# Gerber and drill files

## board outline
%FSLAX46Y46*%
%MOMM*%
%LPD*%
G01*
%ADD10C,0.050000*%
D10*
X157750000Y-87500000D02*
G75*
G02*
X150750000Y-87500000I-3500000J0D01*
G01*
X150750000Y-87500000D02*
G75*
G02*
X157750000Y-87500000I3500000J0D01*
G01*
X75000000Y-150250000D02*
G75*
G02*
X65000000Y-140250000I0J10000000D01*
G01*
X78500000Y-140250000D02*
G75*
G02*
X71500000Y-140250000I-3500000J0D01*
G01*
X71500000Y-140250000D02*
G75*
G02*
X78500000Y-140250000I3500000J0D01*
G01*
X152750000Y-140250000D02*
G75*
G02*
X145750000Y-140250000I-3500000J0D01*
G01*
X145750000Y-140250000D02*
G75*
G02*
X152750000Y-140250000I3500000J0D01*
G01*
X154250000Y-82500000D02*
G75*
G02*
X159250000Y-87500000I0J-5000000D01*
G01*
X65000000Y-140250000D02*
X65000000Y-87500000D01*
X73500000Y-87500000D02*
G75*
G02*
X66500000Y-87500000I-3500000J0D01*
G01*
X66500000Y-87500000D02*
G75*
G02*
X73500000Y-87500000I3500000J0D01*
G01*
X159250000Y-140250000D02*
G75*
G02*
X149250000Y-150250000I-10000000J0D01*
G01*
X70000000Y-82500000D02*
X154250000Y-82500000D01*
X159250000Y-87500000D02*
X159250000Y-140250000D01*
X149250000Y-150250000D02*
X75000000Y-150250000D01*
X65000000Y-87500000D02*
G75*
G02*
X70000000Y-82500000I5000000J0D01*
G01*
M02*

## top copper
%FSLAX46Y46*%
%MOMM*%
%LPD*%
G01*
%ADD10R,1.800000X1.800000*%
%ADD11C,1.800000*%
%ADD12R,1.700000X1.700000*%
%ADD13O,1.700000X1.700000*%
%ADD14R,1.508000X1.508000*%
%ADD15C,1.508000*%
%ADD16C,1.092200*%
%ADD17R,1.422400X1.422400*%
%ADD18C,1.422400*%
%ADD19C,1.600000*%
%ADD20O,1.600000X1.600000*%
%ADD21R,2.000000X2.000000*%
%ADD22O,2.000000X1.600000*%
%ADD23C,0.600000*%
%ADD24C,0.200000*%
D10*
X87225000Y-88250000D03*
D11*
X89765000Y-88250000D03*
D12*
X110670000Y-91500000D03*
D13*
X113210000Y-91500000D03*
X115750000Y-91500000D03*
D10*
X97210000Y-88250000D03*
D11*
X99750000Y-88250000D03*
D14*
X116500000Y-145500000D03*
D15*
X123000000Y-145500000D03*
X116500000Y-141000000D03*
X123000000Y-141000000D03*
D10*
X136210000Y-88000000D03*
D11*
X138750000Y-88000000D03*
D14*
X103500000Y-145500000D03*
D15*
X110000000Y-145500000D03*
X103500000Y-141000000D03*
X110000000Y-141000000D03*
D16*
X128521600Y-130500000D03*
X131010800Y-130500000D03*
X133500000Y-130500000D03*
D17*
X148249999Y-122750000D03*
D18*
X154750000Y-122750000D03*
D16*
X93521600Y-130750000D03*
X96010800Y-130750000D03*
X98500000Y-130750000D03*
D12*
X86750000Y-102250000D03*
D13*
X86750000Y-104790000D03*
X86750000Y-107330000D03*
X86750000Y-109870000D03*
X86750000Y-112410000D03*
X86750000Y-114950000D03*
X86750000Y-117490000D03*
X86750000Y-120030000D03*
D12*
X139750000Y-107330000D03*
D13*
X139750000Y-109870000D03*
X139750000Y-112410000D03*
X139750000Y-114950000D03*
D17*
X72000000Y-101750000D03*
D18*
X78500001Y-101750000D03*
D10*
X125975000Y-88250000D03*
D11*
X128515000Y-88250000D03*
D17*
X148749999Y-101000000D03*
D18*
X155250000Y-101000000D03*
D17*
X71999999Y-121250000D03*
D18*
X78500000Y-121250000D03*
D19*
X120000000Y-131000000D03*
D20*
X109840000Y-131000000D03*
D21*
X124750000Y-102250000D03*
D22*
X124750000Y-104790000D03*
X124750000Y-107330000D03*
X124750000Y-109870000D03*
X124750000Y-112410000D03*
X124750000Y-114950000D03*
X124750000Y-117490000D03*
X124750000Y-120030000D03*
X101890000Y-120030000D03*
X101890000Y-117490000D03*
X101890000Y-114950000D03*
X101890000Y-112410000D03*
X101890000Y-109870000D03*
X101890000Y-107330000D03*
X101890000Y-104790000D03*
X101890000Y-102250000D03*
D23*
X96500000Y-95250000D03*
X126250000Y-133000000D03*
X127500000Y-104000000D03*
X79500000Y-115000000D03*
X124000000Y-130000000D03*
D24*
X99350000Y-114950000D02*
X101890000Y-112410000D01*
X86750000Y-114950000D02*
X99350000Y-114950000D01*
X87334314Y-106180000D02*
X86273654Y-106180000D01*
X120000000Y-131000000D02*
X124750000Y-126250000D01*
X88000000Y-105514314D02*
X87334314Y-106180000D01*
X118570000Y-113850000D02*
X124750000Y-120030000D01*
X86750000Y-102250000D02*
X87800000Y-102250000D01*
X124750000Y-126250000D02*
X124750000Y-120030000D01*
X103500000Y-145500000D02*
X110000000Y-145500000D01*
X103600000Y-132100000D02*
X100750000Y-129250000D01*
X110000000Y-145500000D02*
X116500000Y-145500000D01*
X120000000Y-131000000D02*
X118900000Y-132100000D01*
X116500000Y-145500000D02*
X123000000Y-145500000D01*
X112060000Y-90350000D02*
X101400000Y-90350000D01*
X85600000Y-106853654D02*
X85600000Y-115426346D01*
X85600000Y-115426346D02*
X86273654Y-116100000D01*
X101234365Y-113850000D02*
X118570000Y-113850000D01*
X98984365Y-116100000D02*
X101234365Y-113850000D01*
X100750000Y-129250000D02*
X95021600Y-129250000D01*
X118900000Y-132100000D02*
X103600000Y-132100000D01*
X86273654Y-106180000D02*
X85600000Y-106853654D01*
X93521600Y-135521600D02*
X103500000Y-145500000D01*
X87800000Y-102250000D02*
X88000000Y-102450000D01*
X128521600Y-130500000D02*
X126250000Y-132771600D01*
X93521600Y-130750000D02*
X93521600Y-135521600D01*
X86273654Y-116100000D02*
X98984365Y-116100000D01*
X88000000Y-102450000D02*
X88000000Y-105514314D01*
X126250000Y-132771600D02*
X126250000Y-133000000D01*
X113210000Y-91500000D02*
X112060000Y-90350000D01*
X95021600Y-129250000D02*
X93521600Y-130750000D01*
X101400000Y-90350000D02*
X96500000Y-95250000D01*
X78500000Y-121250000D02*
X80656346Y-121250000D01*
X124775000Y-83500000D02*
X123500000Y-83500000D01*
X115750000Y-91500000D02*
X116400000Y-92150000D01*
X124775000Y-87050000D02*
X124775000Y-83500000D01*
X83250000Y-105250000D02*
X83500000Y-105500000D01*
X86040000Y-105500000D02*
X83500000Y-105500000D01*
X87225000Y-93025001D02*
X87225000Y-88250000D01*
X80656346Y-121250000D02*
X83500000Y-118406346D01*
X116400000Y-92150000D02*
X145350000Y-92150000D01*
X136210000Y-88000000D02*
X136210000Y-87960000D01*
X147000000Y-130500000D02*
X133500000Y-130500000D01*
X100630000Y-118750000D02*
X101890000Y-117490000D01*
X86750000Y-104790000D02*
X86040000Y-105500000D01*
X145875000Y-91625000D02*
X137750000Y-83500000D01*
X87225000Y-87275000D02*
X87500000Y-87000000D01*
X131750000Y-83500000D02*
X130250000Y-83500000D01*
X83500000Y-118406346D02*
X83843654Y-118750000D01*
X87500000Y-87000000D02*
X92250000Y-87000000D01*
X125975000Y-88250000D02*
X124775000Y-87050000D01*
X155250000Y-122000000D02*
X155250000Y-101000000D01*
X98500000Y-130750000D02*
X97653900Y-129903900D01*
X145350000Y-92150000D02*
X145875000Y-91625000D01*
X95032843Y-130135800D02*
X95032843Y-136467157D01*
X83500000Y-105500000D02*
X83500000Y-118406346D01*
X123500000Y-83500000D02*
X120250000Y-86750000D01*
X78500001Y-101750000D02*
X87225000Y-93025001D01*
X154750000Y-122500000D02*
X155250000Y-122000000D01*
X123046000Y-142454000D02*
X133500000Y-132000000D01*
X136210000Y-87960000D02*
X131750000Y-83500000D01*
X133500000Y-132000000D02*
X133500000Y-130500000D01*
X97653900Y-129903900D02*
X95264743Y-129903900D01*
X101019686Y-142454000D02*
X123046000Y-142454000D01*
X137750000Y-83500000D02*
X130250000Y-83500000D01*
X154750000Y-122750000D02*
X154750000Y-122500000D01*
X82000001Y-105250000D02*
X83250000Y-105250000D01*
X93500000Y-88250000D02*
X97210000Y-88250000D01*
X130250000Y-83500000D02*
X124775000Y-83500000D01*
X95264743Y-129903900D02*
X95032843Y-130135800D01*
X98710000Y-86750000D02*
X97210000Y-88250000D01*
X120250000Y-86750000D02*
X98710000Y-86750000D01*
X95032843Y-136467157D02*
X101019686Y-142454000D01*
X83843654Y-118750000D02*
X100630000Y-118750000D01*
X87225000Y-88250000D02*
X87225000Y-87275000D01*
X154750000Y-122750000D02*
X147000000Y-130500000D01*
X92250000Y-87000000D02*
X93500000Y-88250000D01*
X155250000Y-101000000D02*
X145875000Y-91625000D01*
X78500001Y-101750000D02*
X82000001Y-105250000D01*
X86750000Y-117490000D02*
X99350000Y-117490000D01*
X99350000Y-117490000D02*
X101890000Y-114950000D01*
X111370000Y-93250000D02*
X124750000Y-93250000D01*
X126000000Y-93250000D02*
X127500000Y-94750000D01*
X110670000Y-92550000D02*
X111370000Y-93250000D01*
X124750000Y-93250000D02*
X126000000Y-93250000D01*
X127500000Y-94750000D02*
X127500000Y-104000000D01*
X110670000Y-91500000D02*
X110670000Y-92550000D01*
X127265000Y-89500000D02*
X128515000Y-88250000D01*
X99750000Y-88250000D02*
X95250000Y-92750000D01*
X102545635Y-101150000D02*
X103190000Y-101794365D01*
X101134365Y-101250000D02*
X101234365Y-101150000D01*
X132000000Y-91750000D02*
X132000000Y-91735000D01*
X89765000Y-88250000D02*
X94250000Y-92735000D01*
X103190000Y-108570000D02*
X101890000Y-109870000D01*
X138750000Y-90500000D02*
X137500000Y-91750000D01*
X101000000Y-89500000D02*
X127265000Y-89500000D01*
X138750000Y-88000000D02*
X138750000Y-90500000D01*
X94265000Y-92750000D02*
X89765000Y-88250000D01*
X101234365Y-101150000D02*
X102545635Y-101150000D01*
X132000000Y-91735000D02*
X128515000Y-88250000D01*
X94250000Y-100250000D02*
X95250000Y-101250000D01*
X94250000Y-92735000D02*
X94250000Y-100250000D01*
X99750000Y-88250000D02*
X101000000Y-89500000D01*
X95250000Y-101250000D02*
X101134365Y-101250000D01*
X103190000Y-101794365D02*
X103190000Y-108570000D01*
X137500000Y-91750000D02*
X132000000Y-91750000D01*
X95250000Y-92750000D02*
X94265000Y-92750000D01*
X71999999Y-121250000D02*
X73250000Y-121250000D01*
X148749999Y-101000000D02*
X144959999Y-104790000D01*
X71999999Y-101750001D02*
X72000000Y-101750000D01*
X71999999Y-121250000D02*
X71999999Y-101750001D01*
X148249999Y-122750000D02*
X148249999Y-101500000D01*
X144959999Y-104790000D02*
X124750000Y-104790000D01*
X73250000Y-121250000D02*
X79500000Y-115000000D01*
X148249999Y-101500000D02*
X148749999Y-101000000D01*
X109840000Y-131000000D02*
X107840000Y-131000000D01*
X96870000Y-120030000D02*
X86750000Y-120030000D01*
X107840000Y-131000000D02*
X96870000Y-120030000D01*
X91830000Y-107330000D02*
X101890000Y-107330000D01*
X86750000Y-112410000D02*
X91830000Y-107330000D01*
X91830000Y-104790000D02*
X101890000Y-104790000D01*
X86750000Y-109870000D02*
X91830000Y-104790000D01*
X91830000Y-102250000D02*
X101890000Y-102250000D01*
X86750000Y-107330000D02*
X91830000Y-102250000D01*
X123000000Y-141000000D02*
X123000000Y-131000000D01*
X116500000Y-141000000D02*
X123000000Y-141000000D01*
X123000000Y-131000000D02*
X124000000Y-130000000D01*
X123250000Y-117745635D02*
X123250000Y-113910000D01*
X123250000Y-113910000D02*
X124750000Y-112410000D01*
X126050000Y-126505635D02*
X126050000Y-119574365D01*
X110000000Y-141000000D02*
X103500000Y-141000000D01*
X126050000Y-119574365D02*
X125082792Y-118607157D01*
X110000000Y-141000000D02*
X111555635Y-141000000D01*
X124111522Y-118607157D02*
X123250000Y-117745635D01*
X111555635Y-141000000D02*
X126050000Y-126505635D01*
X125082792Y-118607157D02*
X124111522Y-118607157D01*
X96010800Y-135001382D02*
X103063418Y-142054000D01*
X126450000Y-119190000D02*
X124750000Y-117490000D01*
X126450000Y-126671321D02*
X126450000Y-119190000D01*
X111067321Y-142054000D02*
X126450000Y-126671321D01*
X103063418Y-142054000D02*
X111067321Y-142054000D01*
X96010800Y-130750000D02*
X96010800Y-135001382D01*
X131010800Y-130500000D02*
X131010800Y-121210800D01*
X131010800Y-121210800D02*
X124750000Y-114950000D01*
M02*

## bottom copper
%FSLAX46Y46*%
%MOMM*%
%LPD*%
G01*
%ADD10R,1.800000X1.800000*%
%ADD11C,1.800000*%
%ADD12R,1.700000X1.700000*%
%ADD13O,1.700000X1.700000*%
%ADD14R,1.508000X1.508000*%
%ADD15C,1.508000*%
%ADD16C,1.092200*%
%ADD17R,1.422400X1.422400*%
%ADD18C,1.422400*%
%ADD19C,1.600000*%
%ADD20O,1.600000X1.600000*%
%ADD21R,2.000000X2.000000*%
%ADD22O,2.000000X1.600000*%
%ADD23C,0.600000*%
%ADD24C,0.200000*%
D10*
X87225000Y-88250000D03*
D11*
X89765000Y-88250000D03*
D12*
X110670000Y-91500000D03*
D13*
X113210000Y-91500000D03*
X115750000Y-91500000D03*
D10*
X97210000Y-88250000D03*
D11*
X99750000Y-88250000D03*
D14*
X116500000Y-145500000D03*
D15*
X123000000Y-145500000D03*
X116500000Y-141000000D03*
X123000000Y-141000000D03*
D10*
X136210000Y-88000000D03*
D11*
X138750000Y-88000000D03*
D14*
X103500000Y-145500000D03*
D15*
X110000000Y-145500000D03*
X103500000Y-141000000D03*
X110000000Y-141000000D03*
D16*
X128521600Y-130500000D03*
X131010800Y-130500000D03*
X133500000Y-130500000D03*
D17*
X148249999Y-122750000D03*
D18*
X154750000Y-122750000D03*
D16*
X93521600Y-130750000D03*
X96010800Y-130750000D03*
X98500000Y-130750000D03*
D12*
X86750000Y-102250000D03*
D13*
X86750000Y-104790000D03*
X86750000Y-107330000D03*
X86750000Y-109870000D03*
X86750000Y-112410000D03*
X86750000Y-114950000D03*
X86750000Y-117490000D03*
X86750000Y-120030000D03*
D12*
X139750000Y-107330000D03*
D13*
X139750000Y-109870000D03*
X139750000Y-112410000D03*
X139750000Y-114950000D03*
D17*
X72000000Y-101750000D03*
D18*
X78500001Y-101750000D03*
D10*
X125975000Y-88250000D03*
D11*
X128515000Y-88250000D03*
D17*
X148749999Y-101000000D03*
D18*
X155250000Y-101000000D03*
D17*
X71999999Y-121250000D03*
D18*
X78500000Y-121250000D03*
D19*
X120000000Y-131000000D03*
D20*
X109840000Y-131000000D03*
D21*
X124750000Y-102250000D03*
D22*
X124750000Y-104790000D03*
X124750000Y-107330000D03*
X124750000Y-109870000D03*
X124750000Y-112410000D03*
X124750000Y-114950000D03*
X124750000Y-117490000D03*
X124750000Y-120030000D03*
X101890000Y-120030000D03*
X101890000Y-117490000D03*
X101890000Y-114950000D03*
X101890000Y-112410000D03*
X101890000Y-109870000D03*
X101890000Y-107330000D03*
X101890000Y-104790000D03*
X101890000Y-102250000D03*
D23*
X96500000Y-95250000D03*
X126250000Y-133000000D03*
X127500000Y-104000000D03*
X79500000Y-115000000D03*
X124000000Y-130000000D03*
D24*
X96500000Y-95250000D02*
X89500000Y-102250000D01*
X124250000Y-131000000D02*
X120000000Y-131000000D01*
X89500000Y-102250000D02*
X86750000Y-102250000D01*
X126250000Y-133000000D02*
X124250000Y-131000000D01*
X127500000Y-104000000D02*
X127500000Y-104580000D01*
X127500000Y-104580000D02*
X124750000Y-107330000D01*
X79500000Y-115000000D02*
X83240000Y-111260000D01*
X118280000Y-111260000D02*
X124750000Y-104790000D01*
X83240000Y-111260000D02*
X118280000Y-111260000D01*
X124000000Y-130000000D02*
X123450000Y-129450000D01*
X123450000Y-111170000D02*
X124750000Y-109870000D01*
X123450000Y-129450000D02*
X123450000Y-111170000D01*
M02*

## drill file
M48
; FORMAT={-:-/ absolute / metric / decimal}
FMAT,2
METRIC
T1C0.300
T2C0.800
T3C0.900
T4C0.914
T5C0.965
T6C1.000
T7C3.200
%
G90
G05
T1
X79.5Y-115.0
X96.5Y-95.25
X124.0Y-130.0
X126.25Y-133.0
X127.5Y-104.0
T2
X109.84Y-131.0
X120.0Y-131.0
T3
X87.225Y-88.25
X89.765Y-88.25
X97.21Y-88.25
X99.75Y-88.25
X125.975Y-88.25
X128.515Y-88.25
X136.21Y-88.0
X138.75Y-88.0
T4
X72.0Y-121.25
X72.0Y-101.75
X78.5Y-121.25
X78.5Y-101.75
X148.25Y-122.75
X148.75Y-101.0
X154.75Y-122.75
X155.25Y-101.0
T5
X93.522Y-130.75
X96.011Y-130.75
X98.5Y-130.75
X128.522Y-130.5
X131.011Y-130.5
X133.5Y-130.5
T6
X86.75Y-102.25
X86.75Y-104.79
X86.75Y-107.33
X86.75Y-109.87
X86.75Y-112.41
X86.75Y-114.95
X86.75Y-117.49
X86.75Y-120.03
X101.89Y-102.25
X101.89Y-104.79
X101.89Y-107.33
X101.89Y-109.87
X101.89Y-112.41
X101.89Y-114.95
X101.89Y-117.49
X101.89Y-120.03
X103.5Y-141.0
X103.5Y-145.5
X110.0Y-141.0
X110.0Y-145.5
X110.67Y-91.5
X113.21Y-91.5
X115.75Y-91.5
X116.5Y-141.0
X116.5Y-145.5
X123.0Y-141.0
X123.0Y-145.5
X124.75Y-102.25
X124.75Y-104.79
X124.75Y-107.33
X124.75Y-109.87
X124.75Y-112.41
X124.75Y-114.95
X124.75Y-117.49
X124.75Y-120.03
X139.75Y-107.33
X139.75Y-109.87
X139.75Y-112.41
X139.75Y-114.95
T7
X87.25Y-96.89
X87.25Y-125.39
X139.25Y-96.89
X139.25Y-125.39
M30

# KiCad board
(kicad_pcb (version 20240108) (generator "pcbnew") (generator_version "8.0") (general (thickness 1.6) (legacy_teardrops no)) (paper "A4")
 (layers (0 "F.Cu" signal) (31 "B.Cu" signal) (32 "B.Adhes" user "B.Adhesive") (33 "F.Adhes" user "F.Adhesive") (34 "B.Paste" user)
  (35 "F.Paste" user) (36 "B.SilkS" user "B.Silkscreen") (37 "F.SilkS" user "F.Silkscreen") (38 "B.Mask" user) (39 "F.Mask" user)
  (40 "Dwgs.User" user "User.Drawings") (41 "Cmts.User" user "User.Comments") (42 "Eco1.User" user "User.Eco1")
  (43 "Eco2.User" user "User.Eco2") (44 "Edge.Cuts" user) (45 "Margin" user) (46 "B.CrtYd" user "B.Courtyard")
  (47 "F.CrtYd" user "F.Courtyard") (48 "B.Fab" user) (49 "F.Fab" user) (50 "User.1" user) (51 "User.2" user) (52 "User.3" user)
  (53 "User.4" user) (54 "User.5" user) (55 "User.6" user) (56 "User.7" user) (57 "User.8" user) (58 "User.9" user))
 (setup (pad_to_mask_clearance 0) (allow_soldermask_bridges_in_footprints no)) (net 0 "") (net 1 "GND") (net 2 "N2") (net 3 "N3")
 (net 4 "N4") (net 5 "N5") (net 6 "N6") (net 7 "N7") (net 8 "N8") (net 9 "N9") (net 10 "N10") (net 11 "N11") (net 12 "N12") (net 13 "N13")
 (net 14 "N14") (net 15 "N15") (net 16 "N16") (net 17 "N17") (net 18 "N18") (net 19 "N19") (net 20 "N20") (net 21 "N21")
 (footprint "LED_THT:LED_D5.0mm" (layer "F.Cu") (at 87.225 88.25)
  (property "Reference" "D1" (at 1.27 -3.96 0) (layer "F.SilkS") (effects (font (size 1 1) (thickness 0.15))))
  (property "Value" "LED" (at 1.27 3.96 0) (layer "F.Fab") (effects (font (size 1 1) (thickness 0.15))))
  (pad "1" thru_hole rect (at 0 0) (size 1.8 1.8) (drill 0.9) (layers "*.Cu" "*.Mask") (remove_unused_layers no) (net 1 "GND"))
  (pad "2" thru_hole circle (at 2.54 0) (size 1.8 1.8) (drill 0.9) (layers "*.Cu" "*.Mask") (remove_unused_layers no) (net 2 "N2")))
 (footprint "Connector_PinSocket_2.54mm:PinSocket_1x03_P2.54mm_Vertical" (layer "F.Cu") (at 110.67 91.5 90)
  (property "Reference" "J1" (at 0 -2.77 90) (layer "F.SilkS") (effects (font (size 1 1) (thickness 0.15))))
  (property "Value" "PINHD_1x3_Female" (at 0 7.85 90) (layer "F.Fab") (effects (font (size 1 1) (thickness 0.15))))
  (pad "1" thru_hole rect (at 0 0 90) (size 1.7 1.7) (drill 1) (layers "*.Cu" "*.Mask") (remove_unused_layers no) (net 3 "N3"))
  (pad "2" thru_hole oval (at 0 2.54 90) (size 1.7 1.7) (drill 1) (layers "*.Cu" "*.Mask") (remove_unused_layers no) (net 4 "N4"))
  (pad "3" thru_hole oval (at 0 5.08 90) (size 1.7 1.7) (drill 1) (layers "*.Cu" "*.Mask") (remove_unused_layers no) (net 1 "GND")))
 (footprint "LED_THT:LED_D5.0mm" (layer "F.Cu") (at 97.21 88.25)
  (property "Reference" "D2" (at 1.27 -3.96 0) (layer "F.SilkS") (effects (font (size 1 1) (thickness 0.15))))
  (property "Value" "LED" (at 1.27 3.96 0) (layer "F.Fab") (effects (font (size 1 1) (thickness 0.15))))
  (pad "1" thru_hole rect (at 0 0) (size 1.8 1.8) (drill 0.9) (layers "*.Cu" "*.Mask") (remove_unused_layers no) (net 1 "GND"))
  (pad "2" thru_hole circle (at 2.54 0) (size 1.8 1.8) (drill 0.9) (layers "*.Cu" "*.Mask") (remove_unused_layers no) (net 2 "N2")))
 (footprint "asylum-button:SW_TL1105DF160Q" (layer "F.Cu") (at 119.75 143.25)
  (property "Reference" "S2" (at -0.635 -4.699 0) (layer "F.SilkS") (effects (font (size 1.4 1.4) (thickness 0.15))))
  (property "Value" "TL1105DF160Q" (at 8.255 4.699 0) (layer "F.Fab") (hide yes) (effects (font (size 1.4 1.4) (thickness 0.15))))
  (pad "1" thru_hole rect (at -3.25 2.25) (size 1.508 1.508) (drill 1) (layers "*.Cu" "*.Mask") (remove_unused_layers no) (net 4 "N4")
   (solder_mask_margin 0.102))
  (pad "2" thru_hole circle (at 3.25 2.25) (size 1.508 1.508) (drill 1) (layers "*.Cu" "*.Mask") (remove_unused_layers no) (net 4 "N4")
   (solder_mask_margin 0.102))
  (pad "3" thru_hole circle (at -3.25 -2.25) (size 1.508 1.508) (drill 1) (layers "*.Cu" "*.Mask") (remove_unused_layers no) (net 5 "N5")
   (solder_mask_margin 0.102))
  (pad "4" thru_hole circle (at 3.25 -2.25) (size 1.508 1.508) (drill 1) (layers "*.Cu" "*.Mask") (remove_unused_layers no) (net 5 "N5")
   (solder_mask_margin 0.102)))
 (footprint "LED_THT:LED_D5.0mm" (layer "F.Cu") (at 136.21 88)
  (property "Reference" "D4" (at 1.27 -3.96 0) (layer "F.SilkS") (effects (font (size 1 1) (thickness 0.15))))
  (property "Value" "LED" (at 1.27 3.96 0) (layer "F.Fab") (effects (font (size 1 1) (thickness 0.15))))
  (pad "1" thru_hole rect (at 0 0) (size 1.8 1.8) (drill 0.9) (layers "*.Cu" "*.Mask") (remove_unused_layers no) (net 1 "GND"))
  (pad "2" thru_hole circle (at 2.54 0) (size 1.8 1.8) (drill 0.9) (layers "*.Cu" "*.Mask") (remove_unused_layers no) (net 2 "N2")))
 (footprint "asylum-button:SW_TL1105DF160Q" (layer "F.Cu") (at 106.75 143.25)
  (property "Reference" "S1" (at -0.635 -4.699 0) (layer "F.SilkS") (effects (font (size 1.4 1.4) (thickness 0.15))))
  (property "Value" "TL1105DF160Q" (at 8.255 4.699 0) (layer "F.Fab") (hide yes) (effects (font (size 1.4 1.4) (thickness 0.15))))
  (pad "1" thru_hole rect (at -3.25 2.25) (size 1.508 1.508) (drill 1) (layers "*.Cu" "*.Mask") (remove_unused_layers no) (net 4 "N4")
   (solder_mask_margin 0.102))
  (pad "2" thru_hole circle (at 3.25 2.25) (size 1.508 1.508) (drill 1) (layers "*.Cu" "*.Mask") (remove_unused_layers no) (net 4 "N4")
   (solder_mask_margin 0.102))
  (pad "3" thru_hole circle (at -3.25 -2.25) (size 1.508 1.508) (drill 1) (layers "*.Cu" "*.Mask") (remove_unused_layers no) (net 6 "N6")
   (solder_mask_margin 0.102))
  (pad "4" thru_hole circle (at 3.25 -2.25) (size 1.508 1.508) (drill 1) (layers "*.Cu" "*.Mask") (remove_unused_layers no) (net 6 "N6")
   (solder_mask_margin 0.102)))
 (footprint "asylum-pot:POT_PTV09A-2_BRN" (layer "F.Cu") (at 128.5216 130.5)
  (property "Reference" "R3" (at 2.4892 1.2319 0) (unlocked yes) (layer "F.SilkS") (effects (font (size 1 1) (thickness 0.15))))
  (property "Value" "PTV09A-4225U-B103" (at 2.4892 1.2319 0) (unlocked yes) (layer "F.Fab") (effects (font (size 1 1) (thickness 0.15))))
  (pad "1" thru_hole circle (at 0 0) (size 1.0922 1.0922) (drill 0.9652) (layers "*.Cu" "*.Mask") (remove_unused_layers no) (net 4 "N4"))
  (pad "2" thru_hole circle (at 2.4892 0) (size 1.0922 1.0922) (drill 0.9652) (layers "*.Cu" "*.Mask") (remove_unused_layers no)
   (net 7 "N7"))
  (pad "3" thru_hole circle (at 4.9784 0) (size 1.0922 1.0922) (drill 0.9652) (layers "*.Cu" "*.Mask") (remove_unused_layers no)
   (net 1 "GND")))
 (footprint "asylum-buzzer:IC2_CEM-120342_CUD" (layer "F.Cu") (at 148.249999 122.75)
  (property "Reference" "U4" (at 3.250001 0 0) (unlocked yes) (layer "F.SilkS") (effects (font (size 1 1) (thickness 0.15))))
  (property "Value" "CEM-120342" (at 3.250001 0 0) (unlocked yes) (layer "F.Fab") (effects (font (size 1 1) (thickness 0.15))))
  (pad "1" thru_hole rect (at 0 0) (size 1.4224 1.4224) (drill 0.9144) (layers "*.Cu" "*.Mask") (remove_unused_layers no) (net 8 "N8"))
  (pad "2" thru_hole circle (at 6.500001 0) (size 1.4224 1.4224) (drill 0.9144) (layers "*.Cu" "*.Mask") (remove_unused_layers no)
   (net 1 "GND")))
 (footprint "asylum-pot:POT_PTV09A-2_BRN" (layer "F.Cu") (at 93.5216 130.75)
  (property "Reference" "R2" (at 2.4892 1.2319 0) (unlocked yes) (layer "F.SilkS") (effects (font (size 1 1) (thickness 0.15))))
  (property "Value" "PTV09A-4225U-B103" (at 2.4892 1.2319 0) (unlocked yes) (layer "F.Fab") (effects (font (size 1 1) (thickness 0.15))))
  (pad "1" thru_hole circle (at 0 0) (size 1.0922 1.0922) (drill 0.9652) (layers "*.Cu" "*.Mask") (remove_unused_layers no) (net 4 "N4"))
  (pad "2" thru_hole circle (at 2.4892 0) (size 1.0922 1.0922) (drill 0.9652) (layers "*.Cu" "*.Mask") (remove_unused_layers no)
   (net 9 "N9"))
  (pad "3" thru_hole circle (at 4.9784 0) (size 1.0922 1.0922) (drill 0.9652) (layers "*.Cu" "*.Mask") (remove_unused_layers no)
   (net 1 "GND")))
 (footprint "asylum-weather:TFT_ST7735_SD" (layer "F.Cu") (at 106.75 110.89)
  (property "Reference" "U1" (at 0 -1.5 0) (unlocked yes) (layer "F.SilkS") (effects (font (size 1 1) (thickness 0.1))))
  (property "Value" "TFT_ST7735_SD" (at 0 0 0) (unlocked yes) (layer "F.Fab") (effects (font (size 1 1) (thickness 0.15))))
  (pad "" np_thru_hole circle (at -19.5 -14) (size 3.2 3.2) (drill 3.2) (layers "*.Cu" "*.Mask"))
  (pad "" np_thru_hole circle (at -19.5 14.5) (size 3.2 3.2) (drill 3.2) (layers "*.Cu" "*.Mask"))
  (pad "" np_thru_hole circle (at 32.5 -14) (size 3.2 3.2) (drill 3.2) (layers "*.Cu" "*.Mask"))
  (pad "" np_thru_hole circle (at 32.5 14.5) (size 3.2 3.2) (drill 3.2) (layers "*.Cu" "*.Mask"))
  (pad "1" thru_hole rect (at -20 -8.64) (size 1.7 1.7) (drill 1) (layers "*.Cu" "*.Mask") (remove_unused_layers no) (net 4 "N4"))
  (pad "2" thru_hole oval (at -20 -6.1) (size 1.7 1.7) (drill 1) (layers "*.Cu" "*.Mask") (remove_unused_layers no) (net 1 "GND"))
  (pad "3" thru_hole oval (at -20 -3.56) (size 1.7 1.7) (drill 1) (layers "*.Cu" "*.Mask") (remove_unused_layers no) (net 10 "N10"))
  (pad "4" thru_hole oval (at -20 -1.02) (size 1.7 1.7) (drill 1) (layers "*.Cu" "*.Mask") (remove_unused_layers no) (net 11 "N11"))
  (pad "5" thru_hole oval (at -20 1.52) (size 1.7 1.7) (drill 1) (layers "*.Cu" "*.Mask") (remove_unused_layers no) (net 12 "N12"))
  (pad "6" thru_hole oval (at -20 4.06) (size 1.7 1.7) (drill 1) (layers "*.Cu" "*.Mask") (remove_unused_layers no) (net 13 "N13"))
  (pad "7" thru_hole oval (at -20 6.6) (size 1.7 1.7) (drill 1) (layers "*.Cu" "*.Mask") (remove_unused_layers no) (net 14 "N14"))
  (pad "8" thru_hole oval (at -20 9.14) (size 1.7 1.7) (drill 1) (layers "*.Cu" "*.Mask") (remove_unused_layers no) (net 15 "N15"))
  (pad "9" thru_hole rect (at 33 -3.56) (size 1.7 1.7) (drill 1) (layers "*.Cu" "*.Mask") (remove_unused_layers no) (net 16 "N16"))
  (pad "10" thru_hole oval (at 33 -1.02) (size 1.7 1.7) (drill 1) (layers "*.Cu" "*.Mask") (remove_unused_layers no) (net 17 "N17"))
  (pad "11" thru_hole oval (at 33 1.52) (size 1.7 1.7) (drill 1) (layers "*.Cu" "*.Mask") (remove_unused_layers no) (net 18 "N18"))
  (pad "12" thru_hole oval (at 33 4.06) (size 1.7 1.7) (drill 1) (layers "*.Cu" "*.Mask") (remove_unused_layers no) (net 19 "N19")))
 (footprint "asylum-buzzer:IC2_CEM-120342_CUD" (layer "F.Cu") (at 72 101.75)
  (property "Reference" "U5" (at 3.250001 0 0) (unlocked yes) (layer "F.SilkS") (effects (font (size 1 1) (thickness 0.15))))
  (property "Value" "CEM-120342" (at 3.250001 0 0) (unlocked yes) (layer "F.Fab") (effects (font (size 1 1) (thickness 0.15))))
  (pad "1" thru_hole rect (at 0 0) (size 1.4224 1.4224) (drill 0.9144) (layers "*.Cu" "*.Mask") (remove_unused_layers no) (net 8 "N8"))
  (pad "2" thru_hole circle (at 6.500001 0) (size 1.4224 1.4224) (drill 0.9144) (layers "*.Cu" "*.Mask") (remove_unused_layers no)
   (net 1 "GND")))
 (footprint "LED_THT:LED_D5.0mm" (layer "F.Cu") (at 125.975 88.25)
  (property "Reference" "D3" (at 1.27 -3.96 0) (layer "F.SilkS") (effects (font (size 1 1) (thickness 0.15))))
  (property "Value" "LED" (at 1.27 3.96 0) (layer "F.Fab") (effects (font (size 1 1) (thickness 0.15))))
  (pad "1" thru_hole rect (at 0 0) (size 1.8 1.8) (drill 0.9) (layers "*.Cu" "*.Mask") (remove_unused_layers no) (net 1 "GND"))
  (pad "2" thru_hole circle (at 2.54 0) (size 1.8 1.8) (drill 0.9) (layers "*.Cu" "*.Mask") (remove_unused_layers no) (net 2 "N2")))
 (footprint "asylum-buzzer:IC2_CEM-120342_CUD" (layer "F.Cu") (at 148.749999 101)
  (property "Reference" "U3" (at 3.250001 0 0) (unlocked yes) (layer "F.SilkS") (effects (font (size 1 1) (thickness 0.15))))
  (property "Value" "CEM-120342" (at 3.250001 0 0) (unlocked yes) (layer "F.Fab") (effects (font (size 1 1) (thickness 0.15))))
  (pad "1" thru_hole rect (at 0 0) (size 1.4224 1.4224) (drill 0.9144) (layers "*.Cu" "*.Mask") (remove_unused_layers no) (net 8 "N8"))
  (pad "2" thru_hole circle (at 6.500001 0) (size 1.4224 1.4224) (drill 0.9144) (layers "*.Cu" "*.Mask") (remove_unused_layers no)
   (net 1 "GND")))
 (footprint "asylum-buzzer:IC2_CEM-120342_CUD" (layer "F.Cu") (at 71.999999 121.25)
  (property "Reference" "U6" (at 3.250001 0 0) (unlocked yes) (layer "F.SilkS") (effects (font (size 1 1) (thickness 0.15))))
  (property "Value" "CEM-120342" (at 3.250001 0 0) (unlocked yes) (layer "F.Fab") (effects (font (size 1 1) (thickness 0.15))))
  (pad "1" thru_hole rect (at 0 0) (size 1.4224 1.4224) (drill 0.9144) (layers "*.Cu" "*.Mask") (remove_unused_layers no) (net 8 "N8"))
  (pad "2" thru_hole circle (at 6.500001 0) (size 1.4224 1.4224) (drill 0.9144) (layers "*.Cu" "*.Mask") (remove_unused_layers no)
   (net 1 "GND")))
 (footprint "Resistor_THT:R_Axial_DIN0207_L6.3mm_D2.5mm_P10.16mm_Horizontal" (layer "B.Cu") (at 120 131 180)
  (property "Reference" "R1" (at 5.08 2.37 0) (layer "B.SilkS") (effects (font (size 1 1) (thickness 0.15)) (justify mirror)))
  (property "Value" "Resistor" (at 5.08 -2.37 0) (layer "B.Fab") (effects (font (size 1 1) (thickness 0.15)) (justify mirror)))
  (pad "1" thru_hole circle (at 0 0 180) (size 1.6 1.6) (drill 0.8) (layers "*.Cu" "*.Mask") (remove_unused_layers no) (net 4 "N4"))
  (pad "2" thru_hole oval (at 10.16 0 180) (size 1.6 1.6) (drill 0.8) (layers "*.Cu" "*.Mask") (remove_unused_layers no) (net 15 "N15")))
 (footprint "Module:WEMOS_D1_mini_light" (layer "B.Cu") (at 124.75 102.25 180)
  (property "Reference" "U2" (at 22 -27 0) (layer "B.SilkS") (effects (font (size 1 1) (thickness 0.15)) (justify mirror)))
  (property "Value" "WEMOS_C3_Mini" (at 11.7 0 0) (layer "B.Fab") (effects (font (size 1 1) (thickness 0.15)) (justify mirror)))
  (pad "1" thru_hole rect (at 0 0 180) (size 2 2) (drill 1) (layers "*.Cu" "*.Mask") (remove_unused_layers no) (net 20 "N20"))
  (pad "2" thru_hole oval (at 0 -2.54 180) (size 2 1.6) (drill 1) (layers "*.Cu" "*.Mask") (remove_unused_layers no) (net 8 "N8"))
  (pad "3" thru_hole oval (at 0 -5.08 180) (size 2 1.6) (drill 1) (layers "*.Cu" "*.Mask") (remove_unused_layers no) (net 3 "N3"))
  (pad "4" thru_hole oval (at 0 -7.62 180) (size 2 1.6) (drill 1) (layers "*.Cu" "*.Mask") (remove_unused_layers no) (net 5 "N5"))
  (pad "5" thru_hole oval (at 0 -10.16 180) (size 2 1.6) (drill 1) (layers "*.Cu" "*.Mask") (remove_unused_layers no) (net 6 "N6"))
  (pad "6" thru_hole oval (at 0 -12.7 180) (size 2 1.6) (drill 1) (layers "*.Cu" "*.Mask") (remove_unused_layers no) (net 7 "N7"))
  (pad "7" thru_hole oval (at 0 -15.24 180) (size 2 1.6) (drill 1) (layers "*.Cu" "*.Mask") (remove_unused_layers no) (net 9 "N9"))
  (pad "8" thru_hole oval (at 0 -17.78 180) (size 2 1.6) (drill 1) (layers "*.Cu" "*.Mask") (remove_unused_layers no) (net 4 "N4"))
  (pad "9" thru_hole oval (at 22.86 -17.78 180) (size 2 1.6) (drill 1) (layers "*.Cu" "*.Mask") (remove_unused_layers no) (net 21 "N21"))
  (pad "10" thru_hole oval (at 22.86 -15.24 180) (size 2 1.6) (drill 1) (layers "*.Cu" "*.Mask") (remove_unused_layers no) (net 1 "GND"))
  (pad "11" thru_hole oval (at 22.86 -12.7 180) (size 2 1.6) (drill 1) (layers "*.Cu" "*.Mask") (remove_unused_layers no) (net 14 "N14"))
  (pad "12" thru_hole oval (at 22.86 -10.16 180) (size 2 1.6) (drill 1) (layers "*.Cu" "*.Mask") (remove_unused_layers no) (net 13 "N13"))
  (pad "13" thru_hole oval (at 22.86 -7.62 180) (size 2 1.6) (drill 1) (layers "*.Cu" "*.Mask") (remove_unused_layers no) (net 2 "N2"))
  (pad "14" thru_hole oval (at 22.86 -5.08 180) (size 2 1.6) (drill 1) (layers "*.Cu" "*.Mask") (remove_unused_layers no) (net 12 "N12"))
  (pad "15" thru_hole oval (at 22.86 -2.54 180) (size 2 1.6) (drill 1) (layers "*.Cu" "*.Mask") (remove_unused_layers no) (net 11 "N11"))
  (pad "16" thru_hole oval (at 22.86 0 180) (size 2 1.6) (drill 1) (layers "*.Cu" "*.Mask") (remove_unused_layers no) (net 10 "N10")))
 (gr_circle (center 154.25 87.5) (end 154.25 91) (stroke (width 0.05) (type default)) (fill none) (layer "Edge.Cuts"))
 (gr_arc (start 75 150.25) (mid 67.928932 147.321068) (end 65 140.25) (stroke (width 0.05) (type default)) (layer "Edge.Cuts"))
 (gr_circle (center 75 140.25) (end 75 143.75) (stroke (width 0.05) (type default)) (fill none) (layer "Edge.Cuts"))
 (gr_circle (center 149.25 140.25) (end 149.25 143.75) (stroke (width 0.05) (type default)) (fill none) (layer "Edge.Cuts"))
 (gr_arc (start 154.25 82.5) (mid 157.785534 83.964466) (end 159.25 87.5) (stroke (width 0.05) (type default)) (layer "Edge.Cuts"))
 (gr_line (start 65 140.25) (end 65 87.5) (stroke (width 0.05) (type default)) (layer "Edge.Cuts"))
 (gr_circle (center 70 87.5) (end 70 91) (stroke (width 0.05) (type default)) (fill none) (layer "Edge.Cuts"))
 (gr_arc (start 159.25 140.25) (mid 156.321068 147.321068) (end 149.25 150.25) (stroke (width 0.05) (type default)) (layer "Edge.Cuts"))
 (gr_line (start 70 82.5) (end 154.25 82.5) (stroke (width 0.05) (type default)) (layer "Edge.Cuts"))
 (gr_line (start 159.25 87.5) (end 159.25 140.25) (stroke (width 0.05) (type default)) (layer "Edge.Cuts"))
 (gr_line (start 149.25 150.25) (end 75 150.25) (stroke (width 0.05) (type default)) (layer "Edge.Cuts"))
 (gr_arc (start 65 87.5) (mid 66.464466 83.964466) (end 70 82.5) (stroke (width 0.05) (type default)) (layer "Edge.Cuts"))
 (segment (start 99.35 114.95) (end 101.89 112.41) (width 0.2) (layer "F.Cu") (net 13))
 (segment (start 86.75 114.95) (end 99.35 114.95) (width 0.2) (layer "F.Cu") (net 13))
 (segment (start 87.334314 106.18) (end 86.273654 106.18) (width 0.2) (layer "F.Cu") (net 4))
 (segment (start 120 131) (end 124.75 126.25) (width 0.2) (layer "F.Cu") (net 4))
 (segment (start 88 105.514314) (end 87.334314 106.18) (width 0.2) (layer "F.Cu") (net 4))
 (segment (start 118.57 113.85) (end 124.75 120.03) (width 0.2) (layer "F.Cu") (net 4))
 (segment (start 86.75 102.25) (end 87.8 102.25) (width 0.2) (layer "F.Cu") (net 4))
 (segment (start 124.75 126.25) (end 124.75 120.03) (width 0.2) (layer "F.Cu") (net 4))
 (segment (start 103.5 145.5) (end 110 145.5) (width 0.2) (layer "F.Cu") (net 4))
 (segment (start 103.6 132.1) (end 100.75 129.25) (width 0.2) (layer "F.Cu") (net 4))
 (segment (start 110 145.5) (end 116.5 145.5) (width 0.2) (layer "F.Cu") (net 4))
 (segment (start 120 131) (end 118.9 132.1) (width 0.2) (layer "F.Cu") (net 4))
 (segment (start 116.5 145.5) (end 123 145.5) (width 0.2) (layer "F.Cu") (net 4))
 (segment (start 112.06 90.35) (end 101.4 90.35) (width 0.2) (layer "F.Cu") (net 4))
 (segment (start 85.6 106.853654) (end 85.6 115.426346) (width 0.2) (layer "F.Cu") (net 4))
 (segment (start 85.6 115.426346) (end 86.273654 116.1) (width 0.2) (layer "F.Cu") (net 4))
 (segment (start 101.234365 113.85) (end 118.57 113.85) (width 0.2) (layer "F.Cu") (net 4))
 (segment (start 98.984365 116.1) (end 101.234365 113.85) (width 0.2) (layer "F.Cu") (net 4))
 (segment (start 100.75 129.25) (end 95.0216 129.25) (width 0.2) (layer "F.Cu") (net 4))
 (segment (start 118.9 132.1) (end 103.6 132.1) (width 0.2) (layer "F.Cu") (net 4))
 (segment (start 86.273654 106.18) (end 85.6 106.853654) (width 0.2) (layer "F.Cu") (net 4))
 (segment (start 93.5216 135.5216) (end 103.5 145.5) (width 0.2) (layer "F.Cu") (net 4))
 (segment (start 87.8 102.25) (end 88 102.45) (width 0.2) (layer "F.Cu") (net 4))
 (segment (start 128.5216 130.5) (end 126.25 132.7716) (width 0.2) (layer "F.Cu") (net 4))
 (segment (start 93.5216 130.75) (end 93.5216 135.5216) (width 0.2) (layer "F.Cu") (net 4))
 (segment (start 86.273654 116.1) (end 98.984365 116.1) (width 0.2) (layer "F.Cu") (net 4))
 (segment (start 88 102.45) (end 88 105.514314) (width 0.2) (layer "F.Cu") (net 4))
 (segment (start 126.25 132.7716) (end 126.25 133) (width 0.2) (layer "F.Cu") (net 4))
 (segment (start 113.21 91.5) (end 112.06 90.35) (width 0.2) (layer "F.Cu") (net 4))
 (segment (start 95.0216 129.25) (end 93.5216 130.75) (width 0.2) (layer "F.Cu") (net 4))
 (segment (start 101.4 90.35) (end 96.5 95.25) (width 0.2) (layer "F.Cu") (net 4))
 (via (at 96.5 95.25) (size 0.6) (drill 0.3) (layers "F.Cu" "B.Cu") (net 4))
 (via (at 126.25 133) (size 0.6) (drill 0.3) (layers "F.Cu" "B.Cu") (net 4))
 (segment (start 96.5 95.25) (end 89.5 102.25) (width 0.2) (layer "B.Cu") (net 4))
 (segment (start 124.25 131) (end 120 131) (width 0.2) (layer "B.Cu") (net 4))
 (segment (start 89.5 102.25) (end 86.75 102.25) (width 0.2) (layer "B.Cu") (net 4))
 (segment (start 126.25 133) (end 124.25 131) (width 0.2) (layer "B.Cu") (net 4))
 (segment (start 78.5 121.25) (end 80.656346 121.25) (width 0.2) (layer "F.Cu") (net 1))
 (segment (start 124.775 83.5) (end 123.5 83.5) (width 0.2) (layer "F.Cu") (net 1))
 (segment (start 115.75 91.5) (end 116.4 92.15) (width 0.2) (layer "F.Cu") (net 1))
 (segment (start 124.775 87.05) (end 124.775 83.5) (width 0.2) (layer "F.Cu") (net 1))
 (segment (start 83.25 105.25) (end 83.5 105.5) (width 0.2) (layer "F.Cu") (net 1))
 (segment (start 86.04 105.5) (end 83.5 105.5) (width 0.2) (layer "F.Cu") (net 1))
 (segment (start 87.225 93.025001) (end 87.225 88.25) (width 0.2) (layer "F.Cu") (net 1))
 (segment (start 80.656346 121.25) (end 83.5 118.406346) (width 0.2) (layer "F.Cu") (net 1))
 (segment (start 116.4 92.15) (end 145.35 92.15) (width 0.2) (layer "F.Cu") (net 1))
 (segment (start 136.21 88) (end 136.21 87.96) (width 0.2) (layer "F.Cu") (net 1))
 (segment (start 147 130.5) (end 133.5 130.5) (width 0.2) (layer "F.Cu") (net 1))
 (segment (start 100.63 118.75) (end 101.89 117.49) (width 0.2) (layer "F.Cu") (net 1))
 (segment (start 86.75 104.79) (end 86.04 105.5) (width 0.2) (layer "F.Cu") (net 1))
 (segment (start 145.875 91.625) (end 137.75 83.5) (width 0.2) (layer "F.Cu") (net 1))
 (segment (start 87.225 87.275) (end 87.5 87) (width 0.2) (layer "F.Cu") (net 1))
 (segment (start 131.75 83.5) (end 130.25 83.5) (width 0.2) (layer "F.Cu") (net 1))
 (segment (start 83.5 118.406346) (end 83.843654 118.75) (width 0.2) (layer "F.Cu") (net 1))
 (segment (start 87.5 87) (end 92.25 87) (width 0.2) (layer "F.Cu") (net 1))
 (segment (start 125.975 88.25) (end 124.775 87.05) (width 0.2) (layer "F.Cu") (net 1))
 (segment (start 155.25 122) (end 155.25 101) (width 0.2) (layer "F.Cu") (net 1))
 (segment (start 98.5 130.75) (end 97.6539 129.9039) (width 0.2) (layer "F.Cu") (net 1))
 (segment (start 145.35 92.15) (end 145.875 91.625) (width 0.2) (layer "F.Cu") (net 1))
 (segment (start 95.032843 130.1358) (end 95.032843 136.467157) (width 0.2) (layer "F.Cu") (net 1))
 (segment (start 83.5 105.5) (end 83.5 118.406346) (width 0.2) (layer "F.Cu") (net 1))
 (segment (start 123.5 83.5) (end 120.25 86.75) (width 0.2) (layer "F.Cu") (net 1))
 (segment (start 78.500001 101.75) (end 87.225 93.025001) (width 0.2) (layer "F.Cu") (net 1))
 (segment (start 154.75 122.5) (end 155.25 122) (width 0.2) (layer "F.Cu") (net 1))
 (segment (start 123.046 142.454) (end 133.5 132) (width 0.2) (layer "F.Cu") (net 1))
 (segment (start 136.21 87.96) (end 131.75 83.5) (width 0.2) (layer "F.Cu") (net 1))
 (segment (start 133.5 132) (end 133.5 130.5) (width 0.2) (layer "F.Cu") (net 1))
 (segment (start 97.6539 129.9039) (end 95.264743 129.9039) (width 0.2) (layer "F.Cu") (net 1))
 (segment (start 101.019686 142.454) (end 123.046 142.454) (width 0.2) (layer "F.Cu") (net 1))
 (segment (start 137.75 83.5) (end 130.25 83.5) (width 0.2) (layer "F.Cu") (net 1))
 (segment (start 154.75 122.75) (end 154.75 122.5) (width 0.2) (layer "F.Cu") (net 1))
 (segment (start 82.000001 105.25) (end 83.25 105.25) (width 0.2) (layer "F.Cu") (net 1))
 (segment (start 93.5 88.25) (end 97.21 88.25) (width 0.2) (layer "F.Cu") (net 1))
 (segment (start 130.25 83.5) (end 124.775 83.5) (width 0.2) (layer "F.Cu") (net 1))
 (segment (start 95.264743 129.9039) (end 95.032843 130.1358) (width 0.2) (layer "F.Cu") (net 1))
 (segment (start 98.71 86.75) (end 97.21 88.25) (width 0.2) (layer "F.Cu") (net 1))
 (segment (start 120.25 86.75) (end 98.71 86.75) (width 0.2) (layer "F.Cu") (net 1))
 (segment (start 95.032843 136.467157) (end 101.019686 142.454) (width 0.2) (layer "F.Cu") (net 1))
 (segment (start 83.843654 118.75) (end 100.63 118.75) (width 0.2) (layer "F.Cu") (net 1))
 (segment (start 87.225 88.25) (end 87.225 87.275) (width 0.2) (layer "F.Cu") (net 1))
 (segment (start 154.75 122.75) (end 147 130.5) (width 0.2) (layer "F.Cu") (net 1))
 (segment (start 92.25 87) (end 93.5 88.25) (width 0.2) (layer "F.Cu") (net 1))
 (segment (start 155.25 101) (end 145.875 91.625) (width 0.2) (layer "F.Cu") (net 1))
 (segment (start 78.500001 101.75) (end 82.000001 105.25) (width 0.2) (layer "F.Cu") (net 1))
 (segment (start 86.75 117.49) (end 99.35 117.49) (width 0.2) (layer "F.Cu") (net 14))
 (segment (start 99.35 117.49) (end 101.89 114.95) (width 0.2) (layer "F.Cu") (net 14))
 (segment (start 111.37 93.25) (end 124.75 93.25) (width 0.2) (layer "F.Cu") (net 3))
 (segment (start 126 93.25) (end 127.5 94.75) (width 0.2) (layer "F.Cu") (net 3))
 (segment (start 110.67 92.55) (end 111.37 93.25) (width 0.2) (layer "F.Cu") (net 3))
 (segment (start 124.75 93.25) (end 126 93.25) (width 0.2) (layer "F.Cu") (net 3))
 (segment (start 127.5 94.75) (end 127.5 104) (width 0.2) (layer "F.Cu") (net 3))
 (segment (start 110.67 91.5) (end 110.67 92.55) (width 0.2) (layer "F.Cu") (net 3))
 (via (at 127.5 104) (size 0.6) (drill 0.3) (layers "F.Cu" "B.Cu") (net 3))
 (segment (start 127.5 104) (end 127.5 104.58) (width 0.2) (layer "B.Cu") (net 3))
 (segment (start 127.5 104.58) (end 124.75 107.33) (width 0.2) (layer "B.Cu") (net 3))
 (segment (start 127.265 89.5) (end 128.515 88.25) (width 0.2) (layer "F.Cu") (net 2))
 (segment (start 99.75 88.25) (end 95.25 92.75) (width 0.2) (layer "F.Cu") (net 2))
 (segment (start 102.545635 101.15) (end 103.19 101.794365) (width 0.2) (layer "F.Cu") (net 2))
 (segment (start 101.134365 101.25) (end 101.234365 101.15) (width 0.2) (layer "F.Cu") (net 2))
 (segment (start 132 91.75) (end 132 91.735) (width 0.2) (layer "F.Cu") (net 2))
 (segment (start 89.765 88.25) (end 94.25 92.735) (width 0.2) (layer "F.Cu") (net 2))
 (segment (start 103.19 108.57) (end 101.89 109.87) (width 0.2) (layer "F.Cu") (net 2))
 (segment (start 138.75 90.5) (end 137.5 91.75) (width 0.2) (layer "F.Cu") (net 2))
 (segment (start 101 89.5) (end 127.265 89.5) (width 0.2) (layer "F.Cu") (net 2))
 (segment (start 138.75 88) (end 138.75 90.5) (width 0.2) (layer "F.Cu") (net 2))
 (segment (start 94.265 92.75) (end 89.765 88.25) (width 0.2) (layer "F.Cu") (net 2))
 (segment (start 101.234365 101.15) (end 102.545635 101.15) (width 0.2) (layer "F.Cu") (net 2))
 (segment (start 132 91.735) (end 128.515 88.25) (width 0.2) (layer "F.Cu") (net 2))
 (segment (start 94.25 100.25) (end 95.25 101.25) (width 0.2) (layer "F.Cu") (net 2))
 (segment (start 94.25 92.735) (end 94.25 100.25) (width 0.2) (layer "F.Cu") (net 2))
 (segment (start 99.75 88.25) (end 101 89.5) (width 0.2) (layer "F.Cu") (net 2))
 (segment (start 95.25 101.25) (end 101.134365 101.25) (width 0.2) (layer "F.Cu") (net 2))
 (segment (start 103.19 101.794365) (end 103.19 108.57) (width 0.2) (layer "F.Cu") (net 2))
 (segment (start 137.5 91.75) (end 132 91.75) (width 0.2) (layer "F.Cu") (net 2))
 (segment (start 95.25 92.75) (end 94.265 92.75) (width 0.2) (layer "F.Cu") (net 2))
 (segment (start 71.999999 121.25) (end 73.25 121.25) (width 0.2) (layer "F.Cu") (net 8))
 (segment (start 148.749999 101) (end 144.959999 104.79) (width 0.2) (layer "F.Cu") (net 8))
 (segment (start 71.999999 101.750001) (end 72 101.75) (width 0.2) (layer "F.Cu") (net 8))
 (segment (start 71.999999 121.25) (end 71.999999 101.750001) (width 0.2) (layer "F.Cu") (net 8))
 (segment (start 148.249999 122.75) (end 148.249999 101.5) (width 0.2) (layer "F.Cu") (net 8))
 (segment (start 144.959999 104.79) (end 124.75 104.79) (width 0.2) (layer "F.Cu") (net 8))
 (segment (start 73.25 121.25) (end 79.5 115) (width 0.2) (layer "F.Cu") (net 8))
 (segment (start 148.249999 101.5) (end 148.749999 101) (width 0.2) (layer "F.Cu") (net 8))
 (via (at 79.5 115) (size 0.6) (drill 0.3) (layers "F.Cu" "B.Cu") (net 8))
 (segment (start 79.5 115) (end 83.24 111.26) (width 0.2) (layer "B.Cu") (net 8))
 (segment (start 118.28 111.26) (end 124.75 104.79) (width 0.2) (layer "B.Cu") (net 8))
 (segment (start 83.24 111.26) (end 118.28 111.26) (width 0.2) (layer "B.Cu") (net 8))
 (segment (start 109.84 131) (end 107.84 131) (width 0.2) (layer "F.Cu") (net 15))
 (segment (start 96.87 120.03) (end 86.75 120.03) (width 0.2) (layer "F.Cu") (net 15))
 (segment (start 107.84 131) (end 96.87 120.03) (width 0.2) (layer "F.Cu") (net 15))
 (segment (start 91.83 107.33) (end 101.89 107.33) (width 0.2) (layer "F.Cu") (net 12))
 (segment (start 86.75 112.41) (end 91.83 107.33) (width 0.2) (layer "F.Cu") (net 12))
 (segment (start 91.83 104.79) (end 101.89 104.79) (width 0.2) (layer "F.Cu") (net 11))
 (segment (start 86.75 109.87) (end 91.83 104.79) (width 0.2) (layer "F.Cu") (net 11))
 (segment (start 91.83 102.25) (end 101.89 102.25) (width 0.2) (layer "F.Cu") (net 10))
 (segment (start 86.75 107.33) (end 91.83 102.25) (width 0.2) (layer "F.Cu") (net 10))
 (segment (start 123 141) (end 123 131) (width 0.2) (layer "F.Cu") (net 5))
 (segment (start 116.5 141) (end 123 141) (width 0.2) (layer "F.Cu") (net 5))
 (segment (start 123 131) (end 124 130) (width 0.2) (layer "F.Cu") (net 5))
 (via (at 124 130) (size 0.6) (drill 0.3) (layers "F.Cu" "B.Cu") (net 5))
 (segment (start 124 130) (end 123.45 129.45) (width 0.2) (layer "B.Cu") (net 5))
 (segment (start 123.45 111.17) (end 124.75 109.87) (width 0.2) (layer "B.Cu") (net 5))
 (segment (start 123.45 129.45) (end 123.45 111.17) (width 0.2) (layer "B.Cu") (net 5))
 (segment (start 123.25 117.745635) (end 123.25 113.91) (width 0.2) (layer "F.Cu") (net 6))
 (segment (start 123.25 113.91) (end 124.75 112.41) (width 0.2) (layer "F.Cu") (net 6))
 (segment (start 126.05 126.505635) (end 126.05 119.574365) (width 0.2) (layer "F.Cu") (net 6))
 (segment (start 110 141) (end 103.5 141) (width 0.2) (layer "F.Cu") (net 6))
 (segment (start 126.05 119.574365) (end 125.082792 118.607157) (width 0.2) (layer "F.Cu") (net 6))
 (segment (start 110 141) (end 111.555635 141) (width 0.2) (layer "F.Cu") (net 6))
 (segment (start 124.111522 118.607157) (end 123.25 117.745635) (width 0.2) (layer "F.Cu") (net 6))
 (segment (start 111.555635 141) (end 126.05 126.505635) (width 0.2) (layer "F.Cu") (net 6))
 (segment (start 125.082792 118.607157) (end 124.111522 118.607157) (width 0.2) (layer "F.Cu") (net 6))
 (segment (start 96.0108 135.001382) (end 103.063418 142.054) (width 0.2) (layer "F.Cu") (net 9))
 (segment (start 126.45 119.19) (end 124.75 117.49) (width 0.2) (layer "F.Cu") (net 9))
 (segment (start 126.45 126.671321) (end 126.45 119.19) (width 0.2) (layer "F.Cu") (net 9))
 (segment (start 111.067321 142.054) (end 126.45 126.671321) (width 0.2) (layer "F.Cu") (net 9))
 (segment (start 103.063418 142.054) (end 111.067321 142.054) (width 0.2) (layer "F.Cu") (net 9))
 (segment (start 96.0108 130.75) (end 96.0108 135.001382) (width 0.2) (layer "F.Cu") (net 9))
 (segment (start 131.0108 130.5) (end 131.0108 121.2108) (width 0.2) (layer "F.Cu") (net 7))
 (segment (start 131.0108 121.2108) (end 124.75 114.95) (width 0.2) (layer "F.Cu") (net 7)))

